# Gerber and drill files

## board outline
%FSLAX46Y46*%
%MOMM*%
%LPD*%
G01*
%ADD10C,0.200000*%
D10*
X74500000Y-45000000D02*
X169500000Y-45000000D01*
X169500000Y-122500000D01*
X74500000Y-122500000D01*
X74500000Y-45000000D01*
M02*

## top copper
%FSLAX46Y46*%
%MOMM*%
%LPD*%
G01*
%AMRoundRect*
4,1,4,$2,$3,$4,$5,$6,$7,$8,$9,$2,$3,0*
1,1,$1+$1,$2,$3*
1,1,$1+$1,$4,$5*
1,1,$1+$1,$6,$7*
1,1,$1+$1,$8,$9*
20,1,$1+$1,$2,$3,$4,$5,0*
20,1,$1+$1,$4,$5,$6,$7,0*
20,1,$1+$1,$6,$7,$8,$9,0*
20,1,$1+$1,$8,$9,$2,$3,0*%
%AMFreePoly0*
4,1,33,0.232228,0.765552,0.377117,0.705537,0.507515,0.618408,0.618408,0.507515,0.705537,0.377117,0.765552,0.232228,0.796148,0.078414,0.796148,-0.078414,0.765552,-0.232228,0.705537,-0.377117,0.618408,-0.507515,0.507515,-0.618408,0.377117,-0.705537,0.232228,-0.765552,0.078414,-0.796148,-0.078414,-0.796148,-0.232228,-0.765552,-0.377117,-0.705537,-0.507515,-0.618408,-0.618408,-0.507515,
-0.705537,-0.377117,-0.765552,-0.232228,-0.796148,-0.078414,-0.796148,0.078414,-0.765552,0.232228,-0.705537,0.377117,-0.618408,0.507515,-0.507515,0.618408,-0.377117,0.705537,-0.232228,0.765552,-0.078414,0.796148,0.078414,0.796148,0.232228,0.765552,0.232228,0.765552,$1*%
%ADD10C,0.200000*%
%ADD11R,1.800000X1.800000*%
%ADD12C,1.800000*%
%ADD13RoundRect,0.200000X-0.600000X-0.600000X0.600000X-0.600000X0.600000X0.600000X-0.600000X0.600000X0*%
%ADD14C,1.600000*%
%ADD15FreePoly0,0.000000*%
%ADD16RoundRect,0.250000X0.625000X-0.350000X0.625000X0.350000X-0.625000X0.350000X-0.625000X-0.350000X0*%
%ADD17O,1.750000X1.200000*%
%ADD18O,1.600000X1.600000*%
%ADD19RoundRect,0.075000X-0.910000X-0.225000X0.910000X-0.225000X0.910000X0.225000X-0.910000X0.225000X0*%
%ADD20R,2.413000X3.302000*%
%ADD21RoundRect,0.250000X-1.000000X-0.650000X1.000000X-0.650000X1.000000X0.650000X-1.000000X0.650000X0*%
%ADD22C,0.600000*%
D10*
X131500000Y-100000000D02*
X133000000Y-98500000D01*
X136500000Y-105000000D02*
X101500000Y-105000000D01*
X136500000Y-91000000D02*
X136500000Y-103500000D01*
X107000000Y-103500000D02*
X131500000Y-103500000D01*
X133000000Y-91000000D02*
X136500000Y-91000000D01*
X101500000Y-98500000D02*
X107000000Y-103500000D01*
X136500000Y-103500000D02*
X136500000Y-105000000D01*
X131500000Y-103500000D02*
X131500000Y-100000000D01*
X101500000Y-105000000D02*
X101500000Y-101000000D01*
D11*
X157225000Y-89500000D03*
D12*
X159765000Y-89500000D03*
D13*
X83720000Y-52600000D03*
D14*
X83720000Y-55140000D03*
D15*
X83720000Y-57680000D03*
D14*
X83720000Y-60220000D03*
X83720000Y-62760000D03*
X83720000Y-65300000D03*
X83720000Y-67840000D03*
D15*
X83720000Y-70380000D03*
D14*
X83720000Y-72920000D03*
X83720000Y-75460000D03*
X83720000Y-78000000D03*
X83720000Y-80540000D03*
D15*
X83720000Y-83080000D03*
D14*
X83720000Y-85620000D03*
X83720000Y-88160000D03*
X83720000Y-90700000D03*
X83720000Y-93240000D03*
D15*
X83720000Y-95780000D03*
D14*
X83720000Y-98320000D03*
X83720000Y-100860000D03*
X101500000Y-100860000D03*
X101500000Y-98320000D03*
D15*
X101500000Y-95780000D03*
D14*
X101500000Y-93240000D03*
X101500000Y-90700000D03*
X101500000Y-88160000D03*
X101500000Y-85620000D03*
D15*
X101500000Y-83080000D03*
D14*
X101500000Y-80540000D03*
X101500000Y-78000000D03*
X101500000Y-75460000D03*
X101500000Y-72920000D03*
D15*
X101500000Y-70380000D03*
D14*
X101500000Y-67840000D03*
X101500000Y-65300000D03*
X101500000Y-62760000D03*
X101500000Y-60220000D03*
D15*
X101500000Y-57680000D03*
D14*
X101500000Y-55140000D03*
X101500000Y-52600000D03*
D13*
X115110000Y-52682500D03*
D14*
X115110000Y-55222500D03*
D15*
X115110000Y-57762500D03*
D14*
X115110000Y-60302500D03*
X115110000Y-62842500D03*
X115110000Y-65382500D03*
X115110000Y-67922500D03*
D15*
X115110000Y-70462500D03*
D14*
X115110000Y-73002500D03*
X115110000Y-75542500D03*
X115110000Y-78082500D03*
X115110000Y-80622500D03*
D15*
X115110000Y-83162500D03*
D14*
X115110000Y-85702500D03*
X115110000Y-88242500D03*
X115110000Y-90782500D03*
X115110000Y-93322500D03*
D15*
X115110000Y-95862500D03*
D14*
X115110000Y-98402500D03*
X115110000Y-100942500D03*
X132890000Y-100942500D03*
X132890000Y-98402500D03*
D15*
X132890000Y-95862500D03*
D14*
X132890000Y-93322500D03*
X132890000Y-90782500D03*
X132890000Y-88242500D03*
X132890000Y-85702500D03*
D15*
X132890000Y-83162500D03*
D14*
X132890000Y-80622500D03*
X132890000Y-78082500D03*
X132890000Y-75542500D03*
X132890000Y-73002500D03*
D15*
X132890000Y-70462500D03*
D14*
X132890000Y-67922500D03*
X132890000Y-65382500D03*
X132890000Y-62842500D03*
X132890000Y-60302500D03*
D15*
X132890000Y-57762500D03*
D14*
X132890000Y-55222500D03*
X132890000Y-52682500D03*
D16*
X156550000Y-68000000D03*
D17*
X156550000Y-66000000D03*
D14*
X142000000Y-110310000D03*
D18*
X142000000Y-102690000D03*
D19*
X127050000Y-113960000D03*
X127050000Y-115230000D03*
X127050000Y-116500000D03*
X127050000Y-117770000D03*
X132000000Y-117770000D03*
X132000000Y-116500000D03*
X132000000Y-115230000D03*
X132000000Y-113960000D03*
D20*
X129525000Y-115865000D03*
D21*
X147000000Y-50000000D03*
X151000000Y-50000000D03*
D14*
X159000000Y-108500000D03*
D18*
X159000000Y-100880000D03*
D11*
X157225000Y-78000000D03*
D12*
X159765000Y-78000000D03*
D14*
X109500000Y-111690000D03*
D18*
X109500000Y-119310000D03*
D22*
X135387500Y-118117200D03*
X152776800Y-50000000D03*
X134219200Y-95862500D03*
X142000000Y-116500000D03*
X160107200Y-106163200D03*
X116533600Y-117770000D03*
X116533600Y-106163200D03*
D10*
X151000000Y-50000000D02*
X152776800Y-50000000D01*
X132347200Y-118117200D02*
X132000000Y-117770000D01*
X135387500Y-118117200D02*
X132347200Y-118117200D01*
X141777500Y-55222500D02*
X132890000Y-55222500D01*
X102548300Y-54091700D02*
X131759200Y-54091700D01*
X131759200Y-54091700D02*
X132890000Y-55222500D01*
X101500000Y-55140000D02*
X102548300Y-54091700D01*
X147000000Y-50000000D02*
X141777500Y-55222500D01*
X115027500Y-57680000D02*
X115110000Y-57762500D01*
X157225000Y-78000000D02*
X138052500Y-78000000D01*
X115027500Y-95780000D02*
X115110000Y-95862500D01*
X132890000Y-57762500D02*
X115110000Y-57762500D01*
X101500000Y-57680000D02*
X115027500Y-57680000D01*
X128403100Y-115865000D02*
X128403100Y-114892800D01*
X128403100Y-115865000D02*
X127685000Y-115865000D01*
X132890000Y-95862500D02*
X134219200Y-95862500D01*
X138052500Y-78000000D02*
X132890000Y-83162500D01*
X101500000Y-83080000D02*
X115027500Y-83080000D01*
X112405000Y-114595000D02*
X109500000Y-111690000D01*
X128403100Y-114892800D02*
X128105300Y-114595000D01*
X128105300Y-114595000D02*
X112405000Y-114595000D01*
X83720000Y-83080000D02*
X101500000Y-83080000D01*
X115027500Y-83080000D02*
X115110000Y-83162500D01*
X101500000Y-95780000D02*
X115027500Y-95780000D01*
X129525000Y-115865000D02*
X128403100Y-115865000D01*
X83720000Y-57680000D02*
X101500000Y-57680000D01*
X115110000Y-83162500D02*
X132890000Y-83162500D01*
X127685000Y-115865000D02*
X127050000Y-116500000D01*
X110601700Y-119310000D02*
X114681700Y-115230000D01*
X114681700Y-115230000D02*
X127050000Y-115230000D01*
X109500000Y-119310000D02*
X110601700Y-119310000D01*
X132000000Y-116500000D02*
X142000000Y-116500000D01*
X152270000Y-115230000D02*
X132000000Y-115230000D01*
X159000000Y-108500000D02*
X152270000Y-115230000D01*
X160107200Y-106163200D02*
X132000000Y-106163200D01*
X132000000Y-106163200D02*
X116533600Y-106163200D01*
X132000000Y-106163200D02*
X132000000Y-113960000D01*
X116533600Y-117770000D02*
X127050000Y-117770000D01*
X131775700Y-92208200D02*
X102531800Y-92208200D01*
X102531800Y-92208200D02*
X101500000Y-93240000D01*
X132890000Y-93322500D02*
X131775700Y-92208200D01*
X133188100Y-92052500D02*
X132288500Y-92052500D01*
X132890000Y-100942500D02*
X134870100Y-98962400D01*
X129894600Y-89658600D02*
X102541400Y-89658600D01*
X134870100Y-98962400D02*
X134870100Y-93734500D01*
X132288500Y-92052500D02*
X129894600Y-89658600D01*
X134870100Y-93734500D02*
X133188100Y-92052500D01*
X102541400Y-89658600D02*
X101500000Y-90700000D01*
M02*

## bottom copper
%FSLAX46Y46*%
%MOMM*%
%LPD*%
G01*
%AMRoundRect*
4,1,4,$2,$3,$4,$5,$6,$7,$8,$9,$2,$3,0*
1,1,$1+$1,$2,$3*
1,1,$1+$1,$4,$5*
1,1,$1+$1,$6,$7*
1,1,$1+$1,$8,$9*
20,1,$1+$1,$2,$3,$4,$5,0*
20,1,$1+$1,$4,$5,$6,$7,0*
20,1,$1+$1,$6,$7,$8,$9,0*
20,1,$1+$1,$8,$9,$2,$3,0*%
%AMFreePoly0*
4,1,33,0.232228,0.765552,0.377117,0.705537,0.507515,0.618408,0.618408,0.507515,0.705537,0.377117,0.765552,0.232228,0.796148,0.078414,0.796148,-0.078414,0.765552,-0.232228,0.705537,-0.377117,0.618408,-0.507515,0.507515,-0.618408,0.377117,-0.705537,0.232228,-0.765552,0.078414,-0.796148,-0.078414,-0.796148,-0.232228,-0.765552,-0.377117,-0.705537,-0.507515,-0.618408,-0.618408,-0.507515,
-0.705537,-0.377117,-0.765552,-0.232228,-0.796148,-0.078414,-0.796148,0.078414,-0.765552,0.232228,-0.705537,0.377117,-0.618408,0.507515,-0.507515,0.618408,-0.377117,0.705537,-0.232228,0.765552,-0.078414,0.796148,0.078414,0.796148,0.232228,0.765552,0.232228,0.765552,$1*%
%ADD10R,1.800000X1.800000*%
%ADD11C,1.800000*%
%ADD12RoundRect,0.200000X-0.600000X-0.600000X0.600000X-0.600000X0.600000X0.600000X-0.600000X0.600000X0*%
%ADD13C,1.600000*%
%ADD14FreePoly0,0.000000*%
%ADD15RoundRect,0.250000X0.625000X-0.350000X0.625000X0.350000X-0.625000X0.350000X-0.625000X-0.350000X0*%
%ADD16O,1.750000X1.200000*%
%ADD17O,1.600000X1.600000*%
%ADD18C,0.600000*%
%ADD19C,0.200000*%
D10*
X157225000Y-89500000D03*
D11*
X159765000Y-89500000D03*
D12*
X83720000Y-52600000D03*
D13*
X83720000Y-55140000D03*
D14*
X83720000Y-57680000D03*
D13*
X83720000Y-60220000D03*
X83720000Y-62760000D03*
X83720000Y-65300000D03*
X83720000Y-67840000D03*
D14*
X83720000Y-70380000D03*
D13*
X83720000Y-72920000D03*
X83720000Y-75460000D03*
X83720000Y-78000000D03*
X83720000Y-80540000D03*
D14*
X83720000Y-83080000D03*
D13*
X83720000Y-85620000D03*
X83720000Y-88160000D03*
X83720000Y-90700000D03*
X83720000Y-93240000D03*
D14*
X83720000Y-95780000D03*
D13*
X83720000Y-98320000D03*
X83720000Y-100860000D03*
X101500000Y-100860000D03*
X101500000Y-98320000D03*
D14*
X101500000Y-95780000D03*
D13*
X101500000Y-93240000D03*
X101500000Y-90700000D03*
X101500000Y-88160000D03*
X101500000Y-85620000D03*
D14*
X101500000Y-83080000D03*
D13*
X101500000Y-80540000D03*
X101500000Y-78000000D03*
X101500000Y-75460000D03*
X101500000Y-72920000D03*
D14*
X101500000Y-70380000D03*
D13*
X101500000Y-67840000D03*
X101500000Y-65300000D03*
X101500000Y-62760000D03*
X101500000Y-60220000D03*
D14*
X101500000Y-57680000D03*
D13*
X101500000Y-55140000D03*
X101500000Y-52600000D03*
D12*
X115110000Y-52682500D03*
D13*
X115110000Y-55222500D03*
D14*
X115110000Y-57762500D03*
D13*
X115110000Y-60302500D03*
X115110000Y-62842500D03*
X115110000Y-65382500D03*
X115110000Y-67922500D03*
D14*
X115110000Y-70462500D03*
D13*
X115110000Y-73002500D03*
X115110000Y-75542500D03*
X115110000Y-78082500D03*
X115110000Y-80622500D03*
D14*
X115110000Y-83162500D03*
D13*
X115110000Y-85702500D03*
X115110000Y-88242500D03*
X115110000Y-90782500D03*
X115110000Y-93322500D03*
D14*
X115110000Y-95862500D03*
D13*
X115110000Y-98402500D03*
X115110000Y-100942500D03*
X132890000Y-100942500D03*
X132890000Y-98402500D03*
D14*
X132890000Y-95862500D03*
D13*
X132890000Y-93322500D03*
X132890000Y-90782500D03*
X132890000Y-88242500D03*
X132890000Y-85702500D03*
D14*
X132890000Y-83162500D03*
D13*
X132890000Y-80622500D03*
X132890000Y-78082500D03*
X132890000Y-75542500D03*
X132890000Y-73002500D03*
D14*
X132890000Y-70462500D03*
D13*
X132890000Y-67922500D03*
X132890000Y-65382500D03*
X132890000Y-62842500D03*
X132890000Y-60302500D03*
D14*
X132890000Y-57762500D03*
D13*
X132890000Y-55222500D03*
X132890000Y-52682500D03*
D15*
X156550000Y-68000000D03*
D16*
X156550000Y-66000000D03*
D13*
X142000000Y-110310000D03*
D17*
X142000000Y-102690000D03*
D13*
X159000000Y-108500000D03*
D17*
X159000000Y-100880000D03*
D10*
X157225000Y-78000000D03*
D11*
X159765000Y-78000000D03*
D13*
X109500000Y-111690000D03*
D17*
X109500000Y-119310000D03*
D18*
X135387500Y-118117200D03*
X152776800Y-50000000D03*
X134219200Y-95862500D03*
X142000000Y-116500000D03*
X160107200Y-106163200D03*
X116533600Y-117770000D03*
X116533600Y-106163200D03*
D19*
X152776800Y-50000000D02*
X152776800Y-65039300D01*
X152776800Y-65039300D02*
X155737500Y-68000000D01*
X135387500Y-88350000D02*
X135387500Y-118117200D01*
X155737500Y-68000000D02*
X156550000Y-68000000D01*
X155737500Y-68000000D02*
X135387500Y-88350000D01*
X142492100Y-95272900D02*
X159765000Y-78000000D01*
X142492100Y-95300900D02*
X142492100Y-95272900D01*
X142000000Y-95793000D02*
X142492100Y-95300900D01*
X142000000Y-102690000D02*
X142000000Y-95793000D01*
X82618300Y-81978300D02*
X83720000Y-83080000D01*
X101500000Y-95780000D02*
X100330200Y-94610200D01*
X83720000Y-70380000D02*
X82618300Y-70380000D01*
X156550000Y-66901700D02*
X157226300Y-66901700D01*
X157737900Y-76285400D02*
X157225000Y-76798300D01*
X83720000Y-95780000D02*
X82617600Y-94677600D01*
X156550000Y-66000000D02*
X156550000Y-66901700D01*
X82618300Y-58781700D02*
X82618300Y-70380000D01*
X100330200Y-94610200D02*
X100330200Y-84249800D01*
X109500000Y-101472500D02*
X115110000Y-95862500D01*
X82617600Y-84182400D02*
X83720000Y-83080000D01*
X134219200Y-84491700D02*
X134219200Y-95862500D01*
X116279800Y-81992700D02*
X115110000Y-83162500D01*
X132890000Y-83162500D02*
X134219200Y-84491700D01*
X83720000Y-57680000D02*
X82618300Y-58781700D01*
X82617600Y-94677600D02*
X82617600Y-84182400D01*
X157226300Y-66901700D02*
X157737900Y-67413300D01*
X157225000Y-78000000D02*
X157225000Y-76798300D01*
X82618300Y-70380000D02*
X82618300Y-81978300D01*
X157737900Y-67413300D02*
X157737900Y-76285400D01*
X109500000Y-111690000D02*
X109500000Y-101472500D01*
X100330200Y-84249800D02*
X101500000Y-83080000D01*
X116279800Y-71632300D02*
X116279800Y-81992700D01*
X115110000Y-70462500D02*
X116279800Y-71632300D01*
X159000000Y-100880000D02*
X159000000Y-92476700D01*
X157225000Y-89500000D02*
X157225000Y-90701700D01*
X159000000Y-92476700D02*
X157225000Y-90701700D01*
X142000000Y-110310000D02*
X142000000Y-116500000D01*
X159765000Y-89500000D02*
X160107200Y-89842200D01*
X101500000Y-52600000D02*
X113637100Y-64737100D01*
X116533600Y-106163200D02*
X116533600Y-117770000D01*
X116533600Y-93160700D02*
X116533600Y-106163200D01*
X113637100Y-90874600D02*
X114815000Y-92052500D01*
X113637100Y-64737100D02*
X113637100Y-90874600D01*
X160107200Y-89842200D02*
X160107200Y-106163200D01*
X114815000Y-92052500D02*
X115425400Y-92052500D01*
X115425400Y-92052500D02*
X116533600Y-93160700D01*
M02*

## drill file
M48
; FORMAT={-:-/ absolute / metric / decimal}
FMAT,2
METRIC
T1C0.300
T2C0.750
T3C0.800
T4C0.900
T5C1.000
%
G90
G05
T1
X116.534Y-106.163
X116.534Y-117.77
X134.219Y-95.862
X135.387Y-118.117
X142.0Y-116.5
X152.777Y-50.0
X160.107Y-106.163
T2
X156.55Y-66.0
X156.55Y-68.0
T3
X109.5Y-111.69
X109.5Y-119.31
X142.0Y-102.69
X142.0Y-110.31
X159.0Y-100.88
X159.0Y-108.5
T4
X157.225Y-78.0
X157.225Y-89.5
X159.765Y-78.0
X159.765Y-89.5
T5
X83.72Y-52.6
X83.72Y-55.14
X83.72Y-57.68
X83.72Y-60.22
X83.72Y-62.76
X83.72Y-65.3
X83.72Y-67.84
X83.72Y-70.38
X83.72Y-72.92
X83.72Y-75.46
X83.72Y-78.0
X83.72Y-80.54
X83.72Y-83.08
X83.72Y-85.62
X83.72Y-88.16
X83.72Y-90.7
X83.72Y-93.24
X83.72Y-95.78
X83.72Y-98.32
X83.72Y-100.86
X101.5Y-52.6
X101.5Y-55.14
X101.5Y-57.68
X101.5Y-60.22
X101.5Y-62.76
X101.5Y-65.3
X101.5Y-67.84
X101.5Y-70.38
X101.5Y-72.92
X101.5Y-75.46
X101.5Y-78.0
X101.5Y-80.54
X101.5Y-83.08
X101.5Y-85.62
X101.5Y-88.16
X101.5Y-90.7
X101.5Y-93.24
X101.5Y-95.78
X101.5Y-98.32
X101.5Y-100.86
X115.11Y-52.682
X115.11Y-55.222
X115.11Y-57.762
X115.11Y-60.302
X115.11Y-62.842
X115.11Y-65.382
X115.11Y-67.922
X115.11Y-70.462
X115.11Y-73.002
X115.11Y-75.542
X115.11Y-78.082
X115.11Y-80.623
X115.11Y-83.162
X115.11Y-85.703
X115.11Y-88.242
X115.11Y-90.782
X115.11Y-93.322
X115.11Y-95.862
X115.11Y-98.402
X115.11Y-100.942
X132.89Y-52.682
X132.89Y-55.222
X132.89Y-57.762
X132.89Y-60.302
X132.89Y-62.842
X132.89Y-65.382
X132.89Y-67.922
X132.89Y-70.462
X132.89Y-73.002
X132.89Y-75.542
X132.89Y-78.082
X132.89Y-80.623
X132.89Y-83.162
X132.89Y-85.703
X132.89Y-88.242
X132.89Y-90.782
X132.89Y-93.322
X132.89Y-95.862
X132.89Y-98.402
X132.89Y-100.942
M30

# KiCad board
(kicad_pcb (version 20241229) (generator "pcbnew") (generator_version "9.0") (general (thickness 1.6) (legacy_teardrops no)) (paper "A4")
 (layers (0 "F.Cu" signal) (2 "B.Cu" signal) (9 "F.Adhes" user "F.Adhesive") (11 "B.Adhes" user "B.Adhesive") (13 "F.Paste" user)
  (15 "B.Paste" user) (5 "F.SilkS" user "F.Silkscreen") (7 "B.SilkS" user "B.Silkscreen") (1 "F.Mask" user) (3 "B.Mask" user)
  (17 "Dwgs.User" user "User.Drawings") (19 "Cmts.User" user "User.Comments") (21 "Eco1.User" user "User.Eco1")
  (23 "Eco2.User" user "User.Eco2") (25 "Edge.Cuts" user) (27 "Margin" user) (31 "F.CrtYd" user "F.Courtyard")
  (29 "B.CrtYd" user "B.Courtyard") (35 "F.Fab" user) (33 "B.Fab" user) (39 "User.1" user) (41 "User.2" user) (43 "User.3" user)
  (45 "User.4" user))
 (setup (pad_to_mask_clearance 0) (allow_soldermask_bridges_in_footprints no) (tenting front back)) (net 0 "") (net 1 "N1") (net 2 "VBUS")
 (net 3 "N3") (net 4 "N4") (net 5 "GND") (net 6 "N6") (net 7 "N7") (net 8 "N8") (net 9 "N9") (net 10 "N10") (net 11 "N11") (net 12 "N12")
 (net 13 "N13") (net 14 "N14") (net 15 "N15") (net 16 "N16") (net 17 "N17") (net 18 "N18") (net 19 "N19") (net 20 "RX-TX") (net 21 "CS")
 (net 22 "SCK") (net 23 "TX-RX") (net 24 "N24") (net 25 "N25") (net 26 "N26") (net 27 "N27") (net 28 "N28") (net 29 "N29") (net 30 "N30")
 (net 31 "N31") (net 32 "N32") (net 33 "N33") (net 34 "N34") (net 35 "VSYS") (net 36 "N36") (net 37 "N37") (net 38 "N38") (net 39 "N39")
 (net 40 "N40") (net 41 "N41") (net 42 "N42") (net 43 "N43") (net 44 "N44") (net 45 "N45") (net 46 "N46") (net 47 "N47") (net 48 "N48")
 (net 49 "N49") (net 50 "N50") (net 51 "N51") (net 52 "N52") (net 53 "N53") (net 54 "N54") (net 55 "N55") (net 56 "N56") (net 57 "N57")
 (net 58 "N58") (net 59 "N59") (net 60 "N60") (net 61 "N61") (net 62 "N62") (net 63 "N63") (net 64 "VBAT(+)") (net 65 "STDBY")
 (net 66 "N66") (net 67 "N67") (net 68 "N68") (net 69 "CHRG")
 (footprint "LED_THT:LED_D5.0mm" (layer "F.Cu") (at 157.225 89.5)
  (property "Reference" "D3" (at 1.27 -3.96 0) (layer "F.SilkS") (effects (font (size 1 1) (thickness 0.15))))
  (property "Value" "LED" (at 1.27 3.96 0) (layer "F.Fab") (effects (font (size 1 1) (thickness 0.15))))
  (pad "1" thru_hole rect (at 0 0) (size 1.8 1.8) (drill 0.9) (layers "*.Cu" "*.Mask") (remove_unused_layers no) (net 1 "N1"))
  (pad "2" thru_hole circle (at 2.54 0) (size 1.8 1.8) (drill 0.9) (layers "*.Cu" "*.Mask") (remove_unused_layers no) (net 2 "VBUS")))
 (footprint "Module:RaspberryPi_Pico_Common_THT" (layer "F.Cu") (at 83.72 52.6)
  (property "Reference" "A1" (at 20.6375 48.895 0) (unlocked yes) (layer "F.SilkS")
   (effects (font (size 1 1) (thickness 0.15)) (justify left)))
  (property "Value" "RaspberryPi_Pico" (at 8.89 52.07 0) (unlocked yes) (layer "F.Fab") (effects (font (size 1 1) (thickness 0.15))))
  (pad "1" thru_hole roundrect (at 0 0) (size 1.6 1.6) (drill 1) (layers "*.Cu" "*.Mask") (remove_unused_layers no) (roundrect_rratio 0.125)
   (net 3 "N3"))
  (pad "2" thru_hole circle (at 0 2.54) (size 1.6 1.6) (drill 1) (layers "*.Cu" "*.Mask") (remove_unused_layers no) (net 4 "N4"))
  (pad "3" thru_hole custom (at 0 5.08) (size 1.6 1.6) (drill 1) (layers "*.Cu" "*.Mask") (remove_unused_layers no) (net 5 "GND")
   (options (clearance outline) (anchor circle)) (primitives))
  (pad "4" thru_hole circle (at 0 7.62) (size 1.6 1.6) (drill 1) (layers "*.Cu" "*.Mask") (remove_unused_layers no) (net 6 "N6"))
  (pad "5" thru_hole circle (at 0 10.16) (size 1.6 1.6) (drill 1) (layers "*.Cu" "*.Mask") (remove_unused_layers no) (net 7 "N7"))
  (pad "6" thru_hole circle (at 0 12.7) (size 1.6 1.6) (drill 1) (layers "*.Cu" "*.Mask") (remove_unused_layers no) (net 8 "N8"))
  (pad "7" thru_hole circle (at 0 15.24) (size 1.6 1.6) (drill 1) (layers "*.Cu" "*.Mask") (remove_unused_layers no) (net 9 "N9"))
  (pad "8" thru_hole custom (at 0 17.78) (size 1.6 1.6) (drill 1) (layers "*.Cu" "*.Mask") (remove_unused_layers no) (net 5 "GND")
   (options (clearance outline) (anchor circle)) (primitives))
  (pad "9" thru_hole circle (at 0 20.32) (size 1.6 1.6) (drill 1) (layers "*.Cu" "*.Mask") (remove_unused_layers no) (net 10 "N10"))
  (pad "10" thru_hole circle (at 0 22.86) (size 1.6 1.6) (drill 1) (layers "*.Cu" "*.Mask") (remove_unused_layers no) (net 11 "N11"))
  (pad "11" thru_hole circle (at 0 25.4) (size 1.6 1.6) (drill 1) (layers "*.Cu" "*.Mask") (remove_unused_layers no) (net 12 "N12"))
  (pad "12" thru_hole circle (at 0 27.94) (size 1.6 1.6) (drill 1) (layers "*.Cu" "*.Mask") (remove_unused_layers no) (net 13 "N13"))
  (pad "13" thru_hole custom (at 0 30.48) (size 1.6 1.6) (drill 1) (layers "*.Cu" "*.Mask") (remove_unused_layers no) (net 5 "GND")
   (options (clearance outline) (anchor circle)) (primitives))
  (pad "14" thru_hole circle (at 0 33.02) (size 1.6 1.6) (drill 1) (layers "*.Cu" "*.Mask") (remove_unused_layers no) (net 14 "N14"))
  (pad "15" thru_hole circle (at 0 35.56) (size 1.6 1.6) (drill 1) (layers "*.Cu" "*.Mask") (remove_unused_layers no) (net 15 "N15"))
  (pad "16" thru_hole circle (at 0 38.1) (size 1.6 1.6) (drill 1) (layers "*.Cu" "*.Mask") (remove_unused_layers no) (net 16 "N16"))
  (pad "17" thru_hole circle (at 0 40.64) (size 1.6 1.6) (drill 1) (layers "*.Cu" "*.Mask") (remove_unused_layers no) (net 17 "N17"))
  (pad "18" thru_hole custom (at 0 43.18) (size 1.6 1.6) (drill 1) (layers "*.Cu" "*.Mask") (remove_unused_layers no) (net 5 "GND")
   (options (clearance outline) (anchor circle)) (primitives))
  (pad "19" thru_hole circle (at 0 45.72) (size 1.6 1.6) (drill 1) (layers "*.Cu" "*.Mask") (remove_unused_layers no) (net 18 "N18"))
  (pad "20" thru_hole circle (at 0 48.26) (size 1.6 1.6) (drill 1) (layers "*.Cu" "*.Mask") (remove_unused_layers no) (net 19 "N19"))
  (pad "21" thru_hole circle (at 17.78 48.26) (size 1.6 1.6) (drill 1) (layers "*.Cu" "*.Mask") (remove_unused_layers no) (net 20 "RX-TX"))
  (pad "22" thru_hole circle (at 17.78 45.72) (size 1.6 1.6) (drill 1) (layers "*.Cu" "*.Mask") (remove_unused_layers no) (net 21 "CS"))
  (pad "23" thru_hole custom (at 17.78 43.18) (size 1.6 1.6) (drill 1) (layers "*.Cu" "*.Mask") (remove_unused_layers no) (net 5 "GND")
   (options (clearance outline) (anchor circle)) (primitives))
  (pad "24" thru_hole circle (at 17.78 40.64) (size 1.6 1.6) (drill 1) (layers "*.Cu" "*.Mask") (remove_unused_layers no) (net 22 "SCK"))
  (pad "25" thru_hole circle (at 17.78 38.1) (size 1.6 1.6) (drill 1) (layers "*.Cu" "*.Mask") (remove_unused_layers no) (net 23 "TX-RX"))
  (pad "26" thru_hole circle (at 17.78 35.56) (size 1.6 1.6) (drill 1) (layers "*.Cu" "*.Mask") (remove_unused_layers no) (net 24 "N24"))
  (pad "27" thru_hole circle (at 17.78 33.02) (size 1.6 1.6) (drill 1) (layers "*.Cu" "*.Mask") (remove_unused_layers no) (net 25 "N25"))
  (pad "28" thru_hole custom (at 17.78 30.48) (size 1.6 1.6) (drill 1) (layers "*.Cu" "*.Mask") (remove_unused_layers no) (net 5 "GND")
   (options (clearance outline) (anchor circle)) (primitives))
  (pad "29" thru_hole circle (at 17.78 27.94) (size 1.6 1.6) (drill 1) (layers "*.Cu" "*.Mask") (remove_unused_layers no) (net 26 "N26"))
  (pad "30" thru_hole circle (at 17.78 25.4) (size 1.6 1.6) (drill 1) (layers "*.Cu" "*.Mask") (remove_unused_layers no) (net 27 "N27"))
  (pad "31" thru_hole circle (at 17.78 22.86) (size 1.6 1.6) (drill 1) (layers "*.Cu" "*.Mask") (remove_unused_layers no) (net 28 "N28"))
  (pad "32" thru_hole circle (at 17.78 20.32) (size 1.6 1.6) (drill 1) (layers "*.Cu" "*.Mask") (remove_unused_layers no) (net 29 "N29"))
  (pad "33" thru_hole custom (at 17.78 17.78) (size 1.6 1.6) (drill 1) (layers "*.Cu" "*.Mask") (remove_unused_layers no) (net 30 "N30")
   (options (clearance outline) (anchor circle)) (primitives))
  (pad "34" thru_hole circle (at 17.78 15.24) (size 1.6 1.6) (drill 1) (layers "*.Cu" "*.Mask") (remove_unused_layers no) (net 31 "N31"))
  (pad "35" thru_hole circle (at 17.78 12.7) (size 1.6 1.6) (drill 1) (layers "*.Cu" "*.Mask") (remove_unused_layers no) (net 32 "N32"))
  (pad "36" thru_hole circle (at 17.78 10.16) (size 1.6 1.6) (drill 1) (layers "*.Cu" "*.Mask") (remove_unused_layers no) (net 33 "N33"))
  (pad "37" thru_hole circle (at 17.78 7.62) (size 1.6 1.6) (drill 1) (layers "*.Cu" "*.Mask") (remove_unused_layers no) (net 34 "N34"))
  (pad "38" thru_hole custom (at 17.78 5.08) (size 1.6 1.6) (drill 1) (layers "*.Cu" "*.Mask") (remove_unused_layers no) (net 5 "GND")
   (options (clearance outline) (anchor circle)) (primitives))
  (pad "39" thru_hole circle (at 17.78 2.54) (size 1.6 1.6) (drill 1) (layers "*.Cu" "*.Mask") (remove_unused_layers no) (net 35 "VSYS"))
  (pad "40" thru_hole circle (at 17.78 0) (size 1.6 1.6) (drill 1) (layers "*.Cu" "*.Mask") (remove_unused_layers no) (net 2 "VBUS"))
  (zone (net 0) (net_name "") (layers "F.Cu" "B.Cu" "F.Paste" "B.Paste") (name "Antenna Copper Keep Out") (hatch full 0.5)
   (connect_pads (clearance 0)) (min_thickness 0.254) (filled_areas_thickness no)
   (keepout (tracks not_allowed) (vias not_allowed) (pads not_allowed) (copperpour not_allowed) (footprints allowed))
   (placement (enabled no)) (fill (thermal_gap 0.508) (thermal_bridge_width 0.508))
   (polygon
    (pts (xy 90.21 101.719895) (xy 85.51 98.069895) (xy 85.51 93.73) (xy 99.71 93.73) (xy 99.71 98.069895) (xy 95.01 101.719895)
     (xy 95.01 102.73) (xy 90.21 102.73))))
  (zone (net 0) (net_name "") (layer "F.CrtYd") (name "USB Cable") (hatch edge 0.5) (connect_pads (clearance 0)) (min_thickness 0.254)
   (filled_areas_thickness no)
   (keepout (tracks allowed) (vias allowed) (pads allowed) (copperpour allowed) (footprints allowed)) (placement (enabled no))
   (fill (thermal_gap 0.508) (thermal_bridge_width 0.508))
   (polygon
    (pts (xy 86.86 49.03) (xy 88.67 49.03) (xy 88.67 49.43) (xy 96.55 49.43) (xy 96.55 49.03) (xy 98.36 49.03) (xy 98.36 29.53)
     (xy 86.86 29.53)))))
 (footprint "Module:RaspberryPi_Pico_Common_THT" (layer "F.Cu") (at 115.11 52.6825)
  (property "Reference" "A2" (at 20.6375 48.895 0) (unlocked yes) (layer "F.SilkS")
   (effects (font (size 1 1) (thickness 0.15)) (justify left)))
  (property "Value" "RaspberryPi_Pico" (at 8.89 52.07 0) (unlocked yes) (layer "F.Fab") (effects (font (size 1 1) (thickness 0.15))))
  (pad "1" thru_hole roundrect (at 0 0) (size 1.6 1.6) (drill 1) (layers "*.Cu" "*.Mask") (remove_unused_layers no) (roundrect_rratio 0.125)
   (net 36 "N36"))
  (pad "2" thru_hole circle (at 0 2.54) (size 1.6 1.6) (drill 1) (layers "*.Cu" "*.Mask") (remove_unused_layers no) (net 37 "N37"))
  (pad "3" thru_hole custom (at 0 5.08) (size 1.6 1.6) (drill 1) (layers "*.Cu" "*.Mask") (remove_unused_layers no) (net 5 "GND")
   (options (clearance outline) (anchor circle)) (primitives))
  (pad "4" thru_hole circle (at 0 7.62) (size 1.6 1.6) (drill 1) (layers "*.Cu" "*.Mask") (remove_unused_layers no) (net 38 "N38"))
  (pad "5" thru_hole circle (at 0 10.16) (size 1.6 1.6) (drill 1) (layers "*.Cu" "*.Mask") (remove_unused_layers no) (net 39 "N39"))
  (pad "6" thru_hole circle (at 0 12.7) (size 1.6 1.6) (drill 1) (layers "*.Cu" "*.Mask") (remove_unused_layers no) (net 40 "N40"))
  (pad "7" thru_hole circle (at 0 15.24) (size 1.6 1.6) (drill 1) (layers "*.Cu" "*.Mask") (remove_unused_layers no) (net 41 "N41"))
  (pad "8" thru_hole custom (at 0 17.78) (size 1.6 1.6) (drill 1) (layers "*.Cu" "*.Mask") (remove_unused_layers no) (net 5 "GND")
   (options (clearance outline) (anchor circle)) (primitives))
  (pad "9" thru_hole circle (at 0 20.32) (size 1.6 1.6) (drill 1) (layers "*.Cu" "*.Mask") (remove_unused_layers no) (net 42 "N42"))
  (pad "10" thru_hole circle (at 0 22.86) (size 1.6 1.6) (drill 1) (layers "*.Cu" "*.Mask") (remove_unused_layers no) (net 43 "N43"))
  (pad "11" thru_hole circle (at 0 25.4) (size 1.6 1.6) (drill 1) (layers "*.Cu" "*.Mask") (remove_unused_layers no) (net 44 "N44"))
  (pad "12" thru_hole circle (at 0 27.94) (size 1.6 1.6) (drill 1) (layers "*.Cu" "*.Mask") (remove_unused_layers no) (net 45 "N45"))
  (pad "13" thru_hole custom (at 0 30.48) (size 1.6 1.6) (drill 1) (layers "*.Cu" "*.Mask") (remove_unused_layers no) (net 5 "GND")
   (options (clearance outline) (anchor circle)) (primitives))
  (pad "14" thru_hole circle (at 0 33.02) (size 1.6 1.6) (drill 1) (layers "*.Cu" "*.Mask") (remove_unused_layers no) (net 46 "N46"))
  (pad "15" thru_hole circle (at 0 35.56) (size 1.6 1.6) (drill 1) (layers "*.Cu" "*.Mask") (remove_unused_layers no) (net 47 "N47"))
  (pad "16" thru_hole circle (at 0 38.1) (size 1.6 1.6) (drill 1) (layers "*.Cu" "*.Mask") (remove_unused_layers no) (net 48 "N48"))
  (pad "17" thru_hole circle (at 0 40.64) (size 1.6 1.6) (drill 1) (layers "*.Cu" "*.Mask") (remove_unused_layers no) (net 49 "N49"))
  (pad "18" thru_hole custom (at 0 43.18) (size 1.6 1.6) (drill 1) (layers "*.Cu" "*.Mask") (remove_unused_layers no) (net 5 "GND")
   (options (clearance outline) (anchor circle)) (primitives))
  (pad "19" thru_hole circle (at 0 45.72) (size 1.6 1.6) (drill 1) (layers "*.Cu" "*.Mask") (remove_unused_layers no) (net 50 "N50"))
  (pad "20" thru_hole circle (at 0 48.26) (size 1.6 1.6) (drill 1) (layers "*.Cu" "*.Mask") (remove_unused_layers no) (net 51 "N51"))
  (pad "21" thru_hole circle (at 17.78 48.26) (size 1.6 1.6) (drill 1) (layers "*.Cu" "*.Mask") (remove_unused_layers no) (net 23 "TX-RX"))
  (pad "22" thru_hole circle (at 17.78 45.72) (size 1.6 1.6) (drill 1) (layers "*.Cu" "*.Mask") (remove_unused_layers no) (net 21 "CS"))
  (pad "23" thru_hole custom (at 17.78 43.18) (size 1.6 1.6) (drill 1) (layers "*.Cu" "*.Mask") (remove_unused_layers no) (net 5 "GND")
   (options (clearance outline) (anchor circle)) (primitives))
  (pad "24" thru_hole circle (at 17.78 40.64) (size 1.6 1.6) (drill 1) (layers "*.Cu" "*.Mask") (remove_unused_layers no) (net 22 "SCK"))
  (pad "25" thru_hole circle (at 17.78 38.1) (size 1.6 1.6) (drill 1) (layers "*.Cu" "*.Mask") (remove_unused_layers no) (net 20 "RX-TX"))
  (pad "26" thru_hole circle (at 17.78 35.56) (size 1.6 1.6) (drill 1) (layers "*.Cu" "*.Mask") (remove_unused_layers no) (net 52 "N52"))
  (pad "27" thru_hole circle (at 17.78 33.02) (size 1.6 1.6) (drill 1) (layers "*.Cu" "*.Mask") (remove_unused_layers no) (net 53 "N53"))
  (pad "28" thru_hole custom (at 17.78 30.48) (size 1.6 1.6) (drill 1) (layers "*.Cu" "*.Mask") (remove_unused_layers no) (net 5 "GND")
   (options (clearance outline) (anchor circle)) (primitives))
  (pad "29" thru_hole circle (at 17.78 27.94) (size 1.6 1.6) (drill 1) (layers "*.Cu" "*.Mask") (remove_unused_layers no) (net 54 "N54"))
  (pad "30" thru_hole circle (at 17.78 25.4) (size 1.6 1.6) (drill 1) (layers "*.Cu" "*.Mask") (remove_unused_layers no) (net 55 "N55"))
  (pad "31" thru_hole circle (at 17.78 22.86) (size 1.6 1.6) (drill 1) (layers "*.Cu" "*.Mask") (remove_unused_layers no) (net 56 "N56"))
  (pad "32" thru_hole circle (at 17.78 20.32) (size 1.6 1.6) (drill 1) (layers "*.Cu" "*.Mask") (remove_unused_layers no) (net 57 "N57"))
  (pad "33" thru_hole custom (at 17.78 17.78) (size 1.6 1.6) (drill 1) (layers "*.Cu" "*.Mask") (remove_unused_layers no) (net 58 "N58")
   (options (clearance outline) (anchor circle)) (primitives))
  (pad "34" thru_hole circle (at 17.78 15.24) (size 1.6 1.6) (drill 1) (layers "*.Cu" "*.Mask") (remove_unused_layers no) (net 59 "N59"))
  (pad "35" thru_hole circle (at 17.78 12.7) (size 1.6 1.6) (drill 1) (layers "*.Cu" "*.Mask") (remove_unused_layers no) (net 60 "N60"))
  (pad "36" thru_hole circle (at 17.78 10.16) (size 1.6 1.6) (drill 1) (layers "*.Cu" "*.Mask") (remove_unused_layers no) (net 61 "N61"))
  (pad "37" thru_hole circle (at 17.78 7.62) (size 1.6 1.6) (drill 1) (layers "*.Cu" "*.Mask") (remove_unused_layers no) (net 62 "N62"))
  (pad "38" thru_hole custom (at 17.78 5.08) (size 1.6 1.6) (drill 1) (layers "*.Cu" "*.Mask") (remove_unused_layers no) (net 5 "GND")
   (options (clearance outline) (anchor circle)) (primitives))
  (pad "39" thru_hole circle (at 17.78 2.54) (size 1.6 1.6) (drill 1) (layers "*.Cu" "*.Mask") (remove_unused_layers no) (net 35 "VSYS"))
  (pad "40" thru_hole circle (at 17.78 0) (size 1.6 1.6) (drill 1) (layers "*.Cu" "*.Mask") (remove_unused_layers no) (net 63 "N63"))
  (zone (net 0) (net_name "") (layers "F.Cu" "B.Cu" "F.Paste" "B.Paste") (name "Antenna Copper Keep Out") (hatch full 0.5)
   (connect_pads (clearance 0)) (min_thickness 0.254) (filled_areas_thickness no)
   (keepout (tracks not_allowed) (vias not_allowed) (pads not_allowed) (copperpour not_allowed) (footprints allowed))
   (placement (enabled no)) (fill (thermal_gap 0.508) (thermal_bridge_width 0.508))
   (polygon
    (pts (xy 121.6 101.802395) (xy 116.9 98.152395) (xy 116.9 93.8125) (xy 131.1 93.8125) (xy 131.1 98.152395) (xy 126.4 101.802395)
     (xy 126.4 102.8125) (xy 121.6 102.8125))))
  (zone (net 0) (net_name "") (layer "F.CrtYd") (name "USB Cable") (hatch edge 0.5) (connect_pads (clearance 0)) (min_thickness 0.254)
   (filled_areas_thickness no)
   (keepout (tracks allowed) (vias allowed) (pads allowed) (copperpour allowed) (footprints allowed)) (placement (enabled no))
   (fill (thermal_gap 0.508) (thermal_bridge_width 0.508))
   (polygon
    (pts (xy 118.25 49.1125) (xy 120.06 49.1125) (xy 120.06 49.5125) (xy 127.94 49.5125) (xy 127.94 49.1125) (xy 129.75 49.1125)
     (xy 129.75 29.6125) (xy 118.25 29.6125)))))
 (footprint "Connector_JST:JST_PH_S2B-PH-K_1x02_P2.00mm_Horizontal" (layer "F.Cu") (at 156.55 68 90)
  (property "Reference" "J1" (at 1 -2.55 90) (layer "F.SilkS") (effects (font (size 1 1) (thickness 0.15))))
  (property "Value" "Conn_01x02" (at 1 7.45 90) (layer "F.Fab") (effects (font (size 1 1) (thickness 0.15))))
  (pad "1" thru_hole roundrect (at 0 0 90) (size 1.2 1.75) (drill 0.75) (layers "*.Cu" "*.Mask") (remove_unused_layers no)
   (roundrect_rratio 0.208333) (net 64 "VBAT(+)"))
  (pad "2" thru_hole oval (at 2 0 90) (size 1.2 1.75) (drill 0.75) (layers "*.Cu" "*.Mask") (remove_unused_layers no) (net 5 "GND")))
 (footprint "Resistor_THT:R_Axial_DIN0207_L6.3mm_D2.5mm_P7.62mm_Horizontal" (layer "F.Cu") (at 142 110.31 90)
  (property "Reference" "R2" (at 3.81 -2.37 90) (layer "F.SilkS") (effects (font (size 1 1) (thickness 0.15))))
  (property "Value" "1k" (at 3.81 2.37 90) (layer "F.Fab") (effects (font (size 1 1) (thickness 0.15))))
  (pad "1" thru_hole circle (at 0 0 90) (size 1.6 1.6) (drill 0.8) (layers "*.Cu" "*.Mask") (remove_unused_layers no) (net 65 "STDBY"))
  (pad "2" thru_hole oval (at 7.62 0 90) (size 1.6 1.6) (drill 0.8) (layers "*.Cu" "*.Mask") (remove_unused_layers no) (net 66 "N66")))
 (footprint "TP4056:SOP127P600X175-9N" (layer "F.Cu") (at 129.525 115.865)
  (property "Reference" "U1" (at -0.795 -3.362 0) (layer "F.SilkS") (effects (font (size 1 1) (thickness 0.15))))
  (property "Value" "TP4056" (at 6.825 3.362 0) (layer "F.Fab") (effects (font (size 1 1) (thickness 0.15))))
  (pad "1" smd roundrect (at -2.475 -1.905) (size 1.97 0.6) (layers "F.Cu" "F.Mask" "F.Paste") (roundrect_rratio 0.125) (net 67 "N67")
   (solder_mask_margin 0.102))
  (pad "2" smd roundrect (at -2.475 -0.635) (size 1.97 0.6) (layers "F.Cu" "F.Mask" "F.Paste") (roundrect_rratio 0.125) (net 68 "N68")
   (solder_mask_margin 0.102))
  (pad "3" smd roundrect (at -2.475 0.635) (size 1.97 0.6) (layers "F.Cu" "F.Mask" "F.Paste") (roundrect_rratio 0.125) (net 5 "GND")
   (solder_mask_margin 0.102))
  (pad "4" smd roundrect (at -2.475 1.905) (size 1.97 0.6) (layers "F.Cu" "F.Mask" "F.Paste") (roundrect_rratio 0.125) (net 2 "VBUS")
   (solder_mask_margin 0.102))
  (pad "5" smd roundrect (at 2.475 1.905) (size 1.97 0.6) (layers "F.Cu" "F.Mask" "F.Paste") (roundrect_rratio 0.125) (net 64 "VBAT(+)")
   (solder_mask_margin 0.102))
  (pad "6" smd roundrect (at 2.475 0.635) (size 1.97 0.6) (layers "F.Cu" "F.Mask" "F.Paste") (roundrect_rratio 0.125) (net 65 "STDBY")
   (solder_mask_margin 0.102))
  (pad "7" smd roundrect (at 2.475 -0.635) (size 1.97 0.6) (layers "F.Cu" "F.Mask" "F.Paste") (roundrect_rratio 0.125) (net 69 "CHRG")
   (solder_mask_margin 0.102))
  (pad "8" smd roundrect (at 2.475 -1.905) (size 1.97 0.6) (layers "F.Cu" "F.Mask" "F.Paste") (roundrect_rratio 0.125) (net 2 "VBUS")
   (solder_mask_margin 0.102))
  (pad "9" smd rect (at 0 0) (size 2.413 3.302) (layers "F.Cu" "F.Mask") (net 5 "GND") (solder_mask_margin 0.102)))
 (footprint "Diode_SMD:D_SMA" (layer "F.Cu") (at 149 50)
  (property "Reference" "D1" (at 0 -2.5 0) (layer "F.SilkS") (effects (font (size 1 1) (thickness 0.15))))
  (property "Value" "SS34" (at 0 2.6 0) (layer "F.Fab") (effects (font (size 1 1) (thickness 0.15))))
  (pad "1" smd roundrect (at -2 0) (size 2.5 1.8) (layers "F.Cu" "F.Mask" "F.Paste") (roundrect_rratio 0.1388888889) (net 35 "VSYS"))
  (pad "2" smd roundrect (at 2 0) (size 2.5 1.8) (layers "F.Cu" "F.Mask" "F.Paste") (roundrect_rratio 0.1388888889) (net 64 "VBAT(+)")))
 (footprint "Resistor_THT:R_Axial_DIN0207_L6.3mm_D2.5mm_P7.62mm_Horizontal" (layer "F.Cu") (at 159 108.5 90)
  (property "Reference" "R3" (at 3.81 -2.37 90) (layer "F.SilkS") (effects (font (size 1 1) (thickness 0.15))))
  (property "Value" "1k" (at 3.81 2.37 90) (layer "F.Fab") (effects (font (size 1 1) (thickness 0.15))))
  (pad "1" thru_hole circle (at 0 0 90) (size 1.6 1.6) (drill 0.8) (layers "*.Cu" "*.Mask") (remove_unused_layers no) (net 69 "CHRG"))
  (pad "2" thru_hole oval (at 7.62 0 90) (size 1.6 1.6) (drill 0.8) (layers "*.Cu" "*.Mask") (remove_unused_layers no) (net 1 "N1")))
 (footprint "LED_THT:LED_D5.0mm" (layer "F.Cu") (at 157.225 78)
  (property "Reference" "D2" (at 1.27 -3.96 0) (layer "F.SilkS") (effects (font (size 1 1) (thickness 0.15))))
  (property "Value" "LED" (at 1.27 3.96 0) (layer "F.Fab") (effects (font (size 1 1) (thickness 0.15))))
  (pad "1" thru_hole rect (at 0 0) (size 1.8 1.8) (drill 0.9) (layers "*.Cu" "*.Mask") (remove_unused_layers no) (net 5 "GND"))
  (pad "2" thru_hole circle (at 2.54 0) (size 1.8 1.8) (drill 0.9) (layers "*.Cu" "*.Mask") (remove_unused_layers no) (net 66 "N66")))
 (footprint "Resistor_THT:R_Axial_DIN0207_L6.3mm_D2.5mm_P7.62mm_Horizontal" (layer "F.Cu") (at 109.5 111.69 -90)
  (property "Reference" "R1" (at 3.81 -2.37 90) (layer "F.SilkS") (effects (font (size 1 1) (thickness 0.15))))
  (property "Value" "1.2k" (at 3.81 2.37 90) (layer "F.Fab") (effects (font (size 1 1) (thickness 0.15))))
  (pad "1" thru_hole circle (at 0 0 270) (size 1.6 1.6) (drill 0.8) (layers "*.Cu" "*.Mask") (remove_unused_layers no) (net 5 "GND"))
  (pad "2" thru_hole oval (at 7.62 0 270) (size 1.6 1.6) (drill 0.8) (layers "*.Cu" "*.Mask") (remove_unused_layers no) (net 68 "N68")))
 (gr_line (start 131.5 100) (end 133 98.5) (stroke (width 0.2) (type default)) (layer "F.Cu") (net 21))
 (gr_line (start 136.5 105) (end 101.5 105) (stroke (width 0.2) (type default)) (layer "F.Cu") (net 20))
 (gr_line (start 136.5 91) (end 136.5 103.5) (stroke (width 0.2) (type default)) (layer "F.Cu") (net 20))
 (gr_line (start 107 103.5) (end 131.5 103.5) (stroke (width 0.2) (type default)) (layer "F.Cu") (net 21))
 (gr_line (start 133 91) (end 136.5 91) (stroke (width 0.2) (type default)) (layer "F.Cu") (net 20))
 (gr_line (start 101.5 98.5) (end 107 103.5) (stroke (width 0.2) (type default)) (layer "F.Cu") (net 21))
 (gr_line (start 136.5 103.5) (end 136.5 105) (stroke (width 0.2) (type default)) (layer "F.Cu") (net 20))
 (gr_line (start 131.5 103.5) (end 131.5 100) (stroke (width 0.2) (type default)) (layer "F.Cu") (net 21))
 (gr_line (start 101.5 105) (end 101.5 101) (stroke (width 0.2) (type default)) (layer "F.Cu") (net 20))
 (gr_rect (start 74.5 45) (end 169.5 122.5) (stroke (width 0.2) (type solid)) (fill no) (layer "Edge.Cuts"))
 (segment (start 151 50) (end 152.7768 50) (width 0.2) (layer "F.Cu") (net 64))
 (segment (start 132.3472 118.1172) (end 132 117.77) (width 0.2) (layer "F.Cu") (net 64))
 (segment (start 135.3875 118.1172) (end 132.3472 118.1172) (width 0.2) (layer "F.Cu") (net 64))
 (via (at 135.3875 118.1172) (size 0.6) (drill 0.3) (layers "F.Cu" "B.Cu") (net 64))
 (via (at 152.7768 50) (size 0.6) (drill 0.3) (layers "F.Cu" "B.Cu") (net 64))
 (segment (start 152.7768 50) (end 152.7768 65.0393) (width 0.2) (layer "B.Cu") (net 64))
 (segment (start 152.7768 65.0393) (end 155.7375 68) (width 0.2) (layer "B.Cu") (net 64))
 (segment (start 135.3875 88.35) (end 135.3875 118.1172) (width 0.2) (layer "B.Cu") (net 64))
 (segment (start 155.7375 68) (end 156.55 68) (width 0.2) (layer "B.Cu") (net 64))
 (segment (start 155.7375 68) (end 135.3875 88.35) (width 0.2) (layer "B.Cu") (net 64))
 (segment (start 141.7775 55.2225) (end 132.89 55.2225) (width 0.2) (layer "F.Cu") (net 35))
 (segment (start 102.5483 54.0917) (end 131.7592 54.0917) (width 0.2) (layer "F.Cu") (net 35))
 (segment (start 131.7592 54.0917) (end 132.89 55.2225) (width 0.2) (layer "F.Cu") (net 35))
 (segment (start 101.5 55.14) (end 102.5483 54.0917) (width 0.2) (layer "F.Cu") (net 35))
 (segment (start 147 50) (end 141.7775 55.2225) (width 0.2) (layer "F.Cu") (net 35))
 (segment (start 142.4921 95.2729) (end 159.765 78) (width 0.2) (layer "B.Cu") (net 66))
 (segment (start 142.4921 95.3009) (end 142.4921 95.2729) (width 0.2) (layer "B.Cu") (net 66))
 (segment (start 142 95.793) (end 142.4921 95.3009) (width 0.2) (layer "B.Cu") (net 66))
 (segment (start 142 102.69) (end 142 95.793) (width 0.2) (layer "B.Cu") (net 66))
 (segment (start 115.0275 57.68) (end 115.11 57.7625) (width 0.2) (layer "F.Cu") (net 5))
 (segment (start 157.225 78) (end 138.0525 78) (width 0.2) (layer "F.Cu") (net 5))
 (segment (start 115.0275 95.78) (end 115.11 95.8625) (width 0.2) (layer "F.Cu") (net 5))
 (segment (start 132.89 57.7625) (end 115.11 57.7625) (width 0.2) (layer "F.Cu") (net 5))
 (segment (start 101.5 57.68) (end 115.0275 57.68) (width 0.2) (layer "F.Cu") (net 5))
 (segment (start 128.4031 115.865) (end 128.4031 114.8928) (width 0.2) (layer "F.Cu") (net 5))
 (segment (start 128.4031 115.865) (end 127.685 115.865) (width 0.2) (layer "F.Cu") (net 5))
 (segment (start 132.89 95.8625) (end 134.2192 95.8625) (width 0.2) (layer "F.Cu") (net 5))
 (segment (start 138.0525 78) (end 132.89 83.1625) (width 0.2) (layer "F.Cu") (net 5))
 (segment (start 101.5 83.08) (end 115.0275 83.08) (width 0.2) (layer "F.Cu") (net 5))
 (segment (start 112.405 114.595) (end 109.5 111.69) (width 0.2) (layer "F.Cu") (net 5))
 (segment (start 128.4031 114.8928) (end 128.1053 114.595) (width 0.2) (layer "F.Cu") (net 5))
 (segment (start 128.1053 114.595) (end 112.405 114.595) (width 0.2) (layer "F.Cu") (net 5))
 (segment (start 83.72 83.08) (end 101.5 83.08) (width 0.2) (layer "F.Cu") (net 5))
 (segment (start 115.0275 83.08) (end 115.11 83.1625) (width 0.2) (layer "F.Cu") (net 5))
 (segment (start 101.5 95.78) (end 115.0275 95.78) (width 0.2) (layer "F.Cu") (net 5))
 (segment (start 129.525 115.865) (end 128.4031 115.865) (width 0.2) (layer "F.Cu") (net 5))
 (segment (start 83.72 57.68) (end 101.5 57.68) (width 0.2) (layer "F.Cu") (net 5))
 (segment (start 115.11 83.1625) (end 132.89 83.1625) (width 0.2) (layer "F.Cu") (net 5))
 (segment (start 127.685 115.865) (end 127.05 116.5) (width 0.2) (layer "F.Cu") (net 5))
 (via (at 134.2192 95.8625) (size 0.6) (drill 0.3) (layers "F.Cu" "B.Cu") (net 5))
 (segment (start 82.6183 81.9783) (end 83.72 83.08) (width 0.2) (layer "B.Cu") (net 5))
 (segment (start 101.5 95.78) (end 100.3302 94.6102) (width 0.2) (layer "B.Cu") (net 5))
 (segment (start 83.72 70.38) (end 82.6183 70.38) (width 0.2) (layer "B.Cu") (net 5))
 (segment (start 156.55 66.9017) (end 157.2263 66.9017) (width 0.2) (layer "B.Cu") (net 5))
 (segment (start 157.7379 76.2854) (end 157.225 76.7983) (width 0.2) (layer "B.Cu") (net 5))
 (segment (start 83.72 95.78) (end 82.6176 94.6776) (width 0.2) (layer "B.Cu") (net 5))
 (segment (start 156.55 66) (end 156.55 66.9017) (width 0.2) (layer "B.Cu") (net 5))
 (segment (start 82.6183 58.7817) (end 82.6183 70.38) (width 0.2) (layer "B.Cu") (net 5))
 (segment (start 100.3302 94.6102) (end 100.3302 84.2498) (width 0.2) (layer "B.Cu") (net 5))
 (segment (start 109.5 101.4725) (end 115.11 95.8625) (width 0.2) (layer "B.Cu") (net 5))
 (segment (start 82.6176 84.1824) (end 83.72 83.08) (width 0.2) (layer "B.Cu") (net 5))
 (segment (start 134.2192 84.4917) (end 134.2192 95.8625) (width 0.2) (layer "B.Cu") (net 5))
 (segment (start 116.2798 81.9927) (end 115.11 83.1625) (width 0.2) (layer "B.Cu") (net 5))
 (segment (start 132.89 83.1625) (end 134.2192 84.4917) (width 0.2) (layer "B.Cu") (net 5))
 (segment (start 83.72 57.68) (end 82.6183 58.7817) (width 0.2) (layer "B.Cu") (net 5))
 (segment (start 82.6176 94.6776) (end 82.6176 84.1824) (width 0.2) (layer "B.Cu") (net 5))
 (segment (start 157.2263 66.9017) (end 157.7379 67.4133) (width 0.2) (layer "B.Cu") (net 5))
 (segment (start 157.225 78) (end 157.225 76.7983) (width 0.2) (layer "B.Cu") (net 5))
 (segment (start 82.6183 70.38) (end 82.6183 81.9783) (width 0.2) (layer "B.Cu") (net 5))
 (segment (start 157.7379 67.4133) (end 157.7379 76.2854) (width 0.2) (layer "B.Cu") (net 5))
 (segment (start 109.5 111.69) (end 109.5 101.4725) (width 0.2) (layer "B.Cu") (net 5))
 (segment (start 100.3302 84.2498) (end 101.5 83.08) (width 0.2) (layer "B.Cu") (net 5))
 (segment (start 116.2798 71.6323) (end 116.2798 81.9927) (width 0.2) (layer "B.Cu") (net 5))
 (segment (start 115.11 70.4625) (end 116.2798 71.6323) (width 0.2) (layer "B.Cu") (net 5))
 (segment (start 159 100.88) (end 159 92.4767) (width 0.2) (layer "B.Cu") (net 1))
 (segment (start 157.225 89.5) (end 157.225 90.7017) (width 0.2) (layer "B.Cu") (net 1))
 (segment (start 159 92.4767) (end 157.225 90.7017) (width 0.2) (layer "B.Cu") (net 1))
 (segment (start 110.6017 119.31) (end 114.6817 115.23) (width 0.2) (layer "F.Cu") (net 68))
 (segment (start 114.6817 115.23) (end 127.05 115.23) (width 0.2) (layer "F.Cu") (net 68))
 (segment (start 109.5 119.31) (end 110.6017 119.31) (width 0.2) (layer "F.Cu") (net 68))
 (segment (start 132 116.5) (end 142 116.5) (width 0.2) (layer "F.Cu") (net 65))
 (via (at 142 116.5) (size 0.6) (drill 0.3) (layers "F.Cu" "B.Cu") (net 65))
 (segment (start 142 110.31) (end 142 116.5) (width 0.2) (layer "B.Cu") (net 65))
 (segment (start 152.27 115.23) (end 132 115.23) (width 0.2) (layer "F.Cu") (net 69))
 (segment (start 159 108.5) (end 152.27 115.23) (width 0.2) (layer "F.Cu") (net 69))
 (segment (start 160.1072 106.1632) (end 132 106.1632) (width 0.2) (layer "F.Cu") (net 2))
 (segment (start 132 106.1632) (end 116.5336 106.1632) (width 0.2) (layer "F.Cu") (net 2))
 (segment (start 132 106.1632) (end 132 113.96) (width 0.2) (layer "F.Cu") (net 2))
 (segment (start 116.5336 117.77) (end 127.05 117.77) (width 0.2) (layer "F.Cu") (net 2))
 (via (at 160.1072 106.1632) (size 0.6) (drill 0.3) (layers "F.Cu" "B.Cu") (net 2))
 (via (at 116.5336 117.77) (size 0.6) (drill 0.3) (layers "F.Cu" "B.Cu") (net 2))
 (via (at 116.5336 106.1632) (size 0.6) (drill 0.3) (layers "F.Cu" "B.Cu") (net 2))
 (segment (start 159.765 89.5) (end 160.1072 89.8422) (width 0.2) (layer "B.Cu") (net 2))
 (segment (start 101.5 52.6) (end 113.6371 64.7371) (width 0.2) (layer "B.Cu") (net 2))
 (segment (start 116.5336 106.1632) (end 116.5336 117.77) (width 0.2) (layer "B.Cu") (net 2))
 (segment (start 116.5336 93.1607) (end 116.5336 106.1632) (width 0.2) (layer "B.Cu") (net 2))
 (segment (start 113.6371 90.8746) (end 114.815 92.0525) (width 0.2) (layer "B.Cu") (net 2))
 (segment (start 113.6371 64.7371) (end 113.6371 90.8746) (width 0.2) (layer "B.Cu") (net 2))
 (segment (start 160.1072 89.8422) (end 160.1072 106.1632) (width 0.2) (layer "B.Cu") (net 2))
 (segment (start 114.815 92.0525) (end 115.4254 92.0525) (width 0.2) (layer "B.Cu") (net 2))
 (segment (start 115.4254 92.0525) (end 116.5336 93.1607) (width 0.2) (layer "B.Cu") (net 2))
 (segment (start 131.7757 92.2082) (end 102.5318 92.2082) (width 0.2) (layer "F.Cu") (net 22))
 (segment (start 102.5318 92.2082) (end 101.5 93.24) (width 0.2) (layer "F.Cu") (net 22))
 (segment (start 132.89 93.3225) (end 131.7757 92.2082) (width 0.2) (layer "F.Cu") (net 22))
 (segment (start 133.1881 92.0525) (end 132.2885 92.0525) (width 0.2) (layer "F.Cu") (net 23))
 (segment (start 132.89 100.9425) (end 134.8701 98.9624) (width 0.2) (layer "F.Cu") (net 23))
 (segment (start 129.8946 89.6586) (end 102.5414 89.6586) (width 0.2) (layer "F.Cu") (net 23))
 (segment (start 134.8701 98.9624) (end 134.8701 93.7345) (width 0.2) (layer "F.Cu") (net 23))
 (segment (start 132.2885 92.0525) (end 129.8946 89.6586) (width 0.2) (layer "F.Cu") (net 23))
 (segment (start 134.8701 93.7345) (end 133.1881 92.0525) (width 0.2) (layer "F.Cu") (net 23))
 (segment (start 102.5414 89.6586) (end 101.5 90.7) (width 0.2) (layer "F.Cu") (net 23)))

